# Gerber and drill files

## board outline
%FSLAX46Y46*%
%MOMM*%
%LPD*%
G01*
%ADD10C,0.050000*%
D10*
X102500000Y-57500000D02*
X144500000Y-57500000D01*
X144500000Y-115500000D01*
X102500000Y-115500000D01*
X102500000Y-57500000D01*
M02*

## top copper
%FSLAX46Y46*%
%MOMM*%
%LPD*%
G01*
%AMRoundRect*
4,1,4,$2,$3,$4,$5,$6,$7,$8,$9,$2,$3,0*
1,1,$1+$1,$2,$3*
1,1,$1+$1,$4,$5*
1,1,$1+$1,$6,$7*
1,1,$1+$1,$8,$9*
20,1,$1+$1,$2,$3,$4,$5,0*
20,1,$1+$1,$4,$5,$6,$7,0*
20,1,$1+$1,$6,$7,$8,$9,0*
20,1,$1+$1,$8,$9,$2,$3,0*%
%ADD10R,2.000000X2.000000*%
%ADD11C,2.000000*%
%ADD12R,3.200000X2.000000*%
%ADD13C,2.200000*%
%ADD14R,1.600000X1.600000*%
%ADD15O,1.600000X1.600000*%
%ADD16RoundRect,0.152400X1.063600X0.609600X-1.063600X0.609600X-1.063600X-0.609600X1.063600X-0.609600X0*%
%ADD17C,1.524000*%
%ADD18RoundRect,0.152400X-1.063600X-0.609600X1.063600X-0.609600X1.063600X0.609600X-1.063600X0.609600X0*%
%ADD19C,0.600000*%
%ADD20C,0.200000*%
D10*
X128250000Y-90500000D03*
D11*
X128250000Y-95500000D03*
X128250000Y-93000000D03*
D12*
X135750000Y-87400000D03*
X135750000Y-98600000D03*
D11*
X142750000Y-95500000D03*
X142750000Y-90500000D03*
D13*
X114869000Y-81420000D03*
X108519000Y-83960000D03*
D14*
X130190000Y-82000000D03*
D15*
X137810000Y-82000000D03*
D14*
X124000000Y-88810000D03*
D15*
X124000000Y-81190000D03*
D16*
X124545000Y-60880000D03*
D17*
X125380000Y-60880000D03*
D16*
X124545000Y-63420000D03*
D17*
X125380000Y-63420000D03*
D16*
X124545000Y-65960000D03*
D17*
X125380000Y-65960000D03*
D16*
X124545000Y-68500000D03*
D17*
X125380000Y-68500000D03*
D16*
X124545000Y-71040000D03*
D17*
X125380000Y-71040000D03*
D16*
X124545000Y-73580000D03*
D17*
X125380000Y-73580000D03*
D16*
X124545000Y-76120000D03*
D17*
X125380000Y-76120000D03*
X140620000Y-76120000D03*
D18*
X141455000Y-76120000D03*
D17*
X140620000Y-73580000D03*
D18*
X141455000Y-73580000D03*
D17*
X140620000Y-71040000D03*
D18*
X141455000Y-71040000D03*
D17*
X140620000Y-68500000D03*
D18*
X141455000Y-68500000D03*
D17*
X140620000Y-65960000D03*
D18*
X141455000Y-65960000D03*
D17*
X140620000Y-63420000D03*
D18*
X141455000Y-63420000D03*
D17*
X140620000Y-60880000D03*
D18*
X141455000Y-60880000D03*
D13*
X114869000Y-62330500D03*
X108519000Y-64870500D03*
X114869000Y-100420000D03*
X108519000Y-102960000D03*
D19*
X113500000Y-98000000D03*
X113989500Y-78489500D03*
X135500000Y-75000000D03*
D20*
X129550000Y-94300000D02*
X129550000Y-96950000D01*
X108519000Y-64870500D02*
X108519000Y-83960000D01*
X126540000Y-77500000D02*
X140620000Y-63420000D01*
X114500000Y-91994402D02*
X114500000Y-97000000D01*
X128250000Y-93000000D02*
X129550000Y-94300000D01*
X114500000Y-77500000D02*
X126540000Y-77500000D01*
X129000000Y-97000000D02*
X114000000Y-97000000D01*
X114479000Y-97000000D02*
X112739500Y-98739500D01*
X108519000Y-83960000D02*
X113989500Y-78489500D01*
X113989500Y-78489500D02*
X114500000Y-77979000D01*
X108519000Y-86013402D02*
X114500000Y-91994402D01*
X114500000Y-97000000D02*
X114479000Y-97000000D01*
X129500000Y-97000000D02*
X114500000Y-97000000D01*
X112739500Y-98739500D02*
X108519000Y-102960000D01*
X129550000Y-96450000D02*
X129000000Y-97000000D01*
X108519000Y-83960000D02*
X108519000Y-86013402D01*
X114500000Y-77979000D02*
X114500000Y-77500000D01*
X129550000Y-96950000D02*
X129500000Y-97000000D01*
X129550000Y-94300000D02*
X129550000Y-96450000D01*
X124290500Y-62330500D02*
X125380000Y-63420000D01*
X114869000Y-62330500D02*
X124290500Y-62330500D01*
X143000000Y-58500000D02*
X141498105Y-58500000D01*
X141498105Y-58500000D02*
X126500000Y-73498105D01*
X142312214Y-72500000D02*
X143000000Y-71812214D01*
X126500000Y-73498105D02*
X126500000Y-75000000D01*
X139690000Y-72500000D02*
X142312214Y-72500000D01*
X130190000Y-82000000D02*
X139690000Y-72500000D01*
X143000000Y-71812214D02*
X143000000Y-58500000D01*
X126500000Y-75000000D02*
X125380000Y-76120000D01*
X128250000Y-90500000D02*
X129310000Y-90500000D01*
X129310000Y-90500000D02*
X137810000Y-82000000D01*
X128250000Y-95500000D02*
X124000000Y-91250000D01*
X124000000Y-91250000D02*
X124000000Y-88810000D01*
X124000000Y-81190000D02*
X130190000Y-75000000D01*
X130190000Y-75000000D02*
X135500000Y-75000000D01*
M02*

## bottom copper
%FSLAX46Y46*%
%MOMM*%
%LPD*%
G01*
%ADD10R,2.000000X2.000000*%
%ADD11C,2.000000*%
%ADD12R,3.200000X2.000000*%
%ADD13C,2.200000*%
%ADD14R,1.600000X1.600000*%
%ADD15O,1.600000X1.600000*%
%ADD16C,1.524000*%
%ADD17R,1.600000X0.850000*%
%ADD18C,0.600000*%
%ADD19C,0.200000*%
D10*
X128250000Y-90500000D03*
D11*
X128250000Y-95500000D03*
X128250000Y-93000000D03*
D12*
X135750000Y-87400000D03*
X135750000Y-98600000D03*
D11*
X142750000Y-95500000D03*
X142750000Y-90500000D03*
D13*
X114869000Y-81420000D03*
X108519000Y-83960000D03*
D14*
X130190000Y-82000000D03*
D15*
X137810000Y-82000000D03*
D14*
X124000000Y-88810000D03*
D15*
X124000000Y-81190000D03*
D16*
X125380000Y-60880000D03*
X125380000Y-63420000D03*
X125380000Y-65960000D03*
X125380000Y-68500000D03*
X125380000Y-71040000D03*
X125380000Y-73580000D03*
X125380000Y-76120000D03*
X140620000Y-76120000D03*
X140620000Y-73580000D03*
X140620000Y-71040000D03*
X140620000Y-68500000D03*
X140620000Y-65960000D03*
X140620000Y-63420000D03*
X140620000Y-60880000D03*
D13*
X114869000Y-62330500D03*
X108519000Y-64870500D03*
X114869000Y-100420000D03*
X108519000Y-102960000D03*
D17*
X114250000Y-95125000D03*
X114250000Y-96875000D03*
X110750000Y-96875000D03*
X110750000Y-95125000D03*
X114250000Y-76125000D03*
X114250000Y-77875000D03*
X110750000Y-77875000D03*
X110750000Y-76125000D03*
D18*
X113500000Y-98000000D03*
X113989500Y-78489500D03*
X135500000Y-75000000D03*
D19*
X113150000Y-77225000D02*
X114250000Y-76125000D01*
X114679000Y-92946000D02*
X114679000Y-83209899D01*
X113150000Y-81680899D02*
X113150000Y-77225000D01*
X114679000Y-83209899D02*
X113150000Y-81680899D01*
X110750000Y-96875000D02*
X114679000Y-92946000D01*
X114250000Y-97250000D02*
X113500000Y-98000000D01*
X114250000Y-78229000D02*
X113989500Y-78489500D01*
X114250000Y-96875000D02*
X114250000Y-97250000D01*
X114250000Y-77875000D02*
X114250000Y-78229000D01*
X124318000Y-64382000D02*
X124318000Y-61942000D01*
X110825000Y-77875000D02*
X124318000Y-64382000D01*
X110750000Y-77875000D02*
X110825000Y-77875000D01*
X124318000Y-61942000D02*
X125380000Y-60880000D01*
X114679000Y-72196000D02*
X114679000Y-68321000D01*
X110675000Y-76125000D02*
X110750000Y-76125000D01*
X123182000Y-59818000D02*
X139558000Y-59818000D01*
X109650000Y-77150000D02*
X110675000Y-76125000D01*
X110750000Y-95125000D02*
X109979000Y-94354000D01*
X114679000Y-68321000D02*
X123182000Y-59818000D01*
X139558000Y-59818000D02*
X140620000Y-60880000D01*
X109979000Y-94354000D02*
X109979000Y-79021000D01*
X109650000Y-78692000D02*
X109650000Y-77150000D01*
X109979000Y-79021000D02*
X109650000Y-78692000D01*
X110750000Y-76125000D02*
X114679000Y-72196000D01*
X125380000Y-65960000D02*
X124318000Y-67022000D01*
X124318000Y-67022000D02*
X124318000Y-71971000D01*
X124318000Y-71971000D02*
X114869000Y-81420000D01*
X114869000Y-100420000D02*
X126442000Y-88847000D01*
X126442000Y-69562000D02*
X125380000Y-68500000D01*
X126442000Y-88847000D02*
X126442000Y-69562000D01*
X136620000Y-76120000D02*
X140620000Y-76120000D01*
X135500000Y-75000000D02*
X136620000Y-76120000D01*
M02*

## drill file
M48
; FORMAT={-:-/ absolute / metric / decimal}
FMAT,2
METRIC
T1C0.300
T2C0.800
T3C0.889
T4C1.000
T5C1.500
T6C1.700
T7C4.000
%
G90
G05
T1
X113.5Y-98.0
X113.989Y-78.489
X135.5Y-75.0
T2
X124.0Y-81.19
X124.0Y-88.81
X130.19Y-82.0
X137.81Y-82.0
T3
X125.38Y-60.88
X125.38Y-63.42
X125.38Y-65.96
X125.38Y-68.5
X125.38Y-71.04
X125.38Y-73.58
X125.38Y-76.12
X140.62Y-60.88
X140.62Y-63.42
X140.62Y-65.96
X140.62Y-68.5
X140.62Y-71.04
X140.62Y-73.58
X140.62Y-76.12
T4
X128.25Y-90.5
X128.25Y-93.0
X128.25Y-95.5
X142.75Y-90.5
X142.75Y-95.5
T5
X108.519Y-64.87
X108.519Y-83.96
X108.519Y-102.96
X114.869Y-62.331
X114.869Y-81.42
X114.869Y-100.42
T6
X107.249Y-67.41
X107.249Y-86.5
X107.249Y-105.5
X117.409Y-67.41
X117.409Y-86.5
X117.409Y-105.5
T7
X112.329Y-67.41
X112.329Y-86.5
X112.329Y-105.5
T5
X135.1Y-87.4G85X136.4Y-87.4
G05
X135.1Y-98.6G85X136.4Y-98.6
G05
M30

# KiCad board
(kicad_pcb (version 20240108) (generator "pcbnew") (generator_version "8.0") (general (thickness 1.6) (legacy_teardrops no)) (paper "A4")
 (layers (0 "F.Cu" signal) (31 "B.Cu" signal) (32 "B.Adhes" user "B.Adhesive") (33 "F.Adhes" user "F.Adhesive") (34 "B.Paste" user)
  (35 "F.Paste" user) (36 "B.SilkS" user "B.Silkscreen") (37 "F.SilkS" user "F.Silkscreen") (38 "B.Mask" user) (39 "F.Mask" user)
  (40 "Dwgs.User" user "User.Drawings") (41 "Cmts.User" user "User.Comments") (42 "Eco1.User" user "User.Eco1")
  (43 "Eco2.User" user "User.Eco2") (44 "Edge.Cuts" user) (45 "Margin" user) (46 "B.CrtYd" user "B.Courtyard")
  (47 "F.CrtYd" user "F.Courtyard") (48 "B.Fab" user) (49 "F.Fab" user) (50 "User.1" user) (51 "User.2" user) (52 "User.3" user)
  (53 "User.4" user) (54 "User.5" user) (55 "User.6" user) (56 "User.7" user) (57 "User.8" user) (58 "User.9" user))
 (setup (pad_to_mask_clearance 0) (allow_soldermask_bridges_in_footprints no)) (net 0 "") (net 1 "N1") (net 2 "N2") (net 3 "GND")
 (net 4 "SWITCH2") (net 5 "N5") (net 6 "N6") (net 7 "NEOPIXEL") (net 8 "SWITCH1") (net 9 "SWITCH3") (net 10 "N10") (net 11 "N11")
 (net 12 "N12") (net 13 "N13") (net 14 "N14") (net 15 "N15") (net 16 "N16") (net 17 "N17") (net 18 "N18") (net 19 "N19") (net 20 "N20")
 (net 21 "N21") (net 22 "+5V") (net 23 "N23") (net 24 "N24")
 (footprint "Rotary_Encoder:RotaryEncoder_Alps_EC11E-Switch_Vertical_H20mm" (layer "F.Cu") (at 128.25 90.5)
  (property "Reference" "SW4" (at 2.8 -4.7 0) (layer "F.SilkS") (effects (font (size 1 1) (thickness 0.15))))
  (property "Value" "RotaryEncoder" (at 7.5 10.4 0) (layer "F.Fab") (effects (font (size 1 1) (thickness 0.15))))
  (pad "A" thru_hole rect (at 0 0) (size 2 2) (drill 1) (layers "*.Cu" "*.Mask") (remove_unused_layers no) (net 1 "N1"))
  (pad "B" thru_hole circle (at 0 5) (size 2 2) (drill 1) (layers "*.Cu" "*.Mask") (remove_unused_layers no) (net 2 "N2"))
  (pad "C" thru_hole circle (at 0 2.5) (size 2 2) (drill 1) (layers "*.Cu" "*.Mask") (remove_unused_layers no) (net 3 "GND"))
  (pad "MP" thru_hole rect (at 7.5 -3.1) (size 3.2 2) (drill oval 2.8 1.5) (layers "*.Cu" "*.Mask") (remove_unused_layers no))
  (pad "MP" thru_hole rect (at 7.5 8.1) (size 3.2 2) (drill oval 2.8 1.5) (layers "*.Cu" "*.Mask") (remove_unused_layers no))
  (pad "S1" thru_hole circle (at 14.5 5) (size 2 2) (drill 1) (layers "*.Cu" "*.Mask") (remove_unused_layers no))
  (pad "S2" thru_hole circle (at 14.5 0) (size 2 2) (drill 1) (layers "*.Cu" "*.Mask") (remove_unused_layers no)))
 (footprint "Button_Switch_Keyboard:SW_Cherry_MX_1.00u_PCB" (layer "F.Cu") (at 114.869 81.42)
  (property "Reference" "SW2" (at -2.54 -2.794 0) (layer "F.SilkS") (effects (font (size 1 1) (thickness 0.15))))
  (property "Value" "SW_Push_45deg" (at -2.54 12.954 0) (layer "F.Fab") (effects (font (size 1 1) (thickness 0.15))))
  (pad "" np_thru_hole circle (at -7.62 5.08) (size 1.7 1.7) (drill 1.7) (layers "*.Cu" "*.Mask"))
  (pad "" np_thru_hole circle (at -2.54 5.08) (size 4 4) (drill 4) (layers "*.Cu" "*.Mask"))
  (pad "" np_thru_hole circle (at 2.54 5.08) (size 1.7 1.7) (drill 1.7) (layers "*.Cu" "*.Mask"))
  (pad "1" thru_hole circle (at 0 0) (size 2.2 2.2) (drill 1.5) (layers "*.Cu" "*.Mask") (remove_unused_layers no) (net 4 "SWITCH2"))
  (pad "2" thru_hole circle (at -6.35 2.54) (size 2.2 2.2) (drill 1.5) (layers "*.Cu" "*.Mask") (remove_unused_layers no) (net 3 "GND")))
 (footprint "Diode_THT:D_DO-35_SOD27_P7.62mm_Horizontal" (layer "F.Cu") (at 130.19 82)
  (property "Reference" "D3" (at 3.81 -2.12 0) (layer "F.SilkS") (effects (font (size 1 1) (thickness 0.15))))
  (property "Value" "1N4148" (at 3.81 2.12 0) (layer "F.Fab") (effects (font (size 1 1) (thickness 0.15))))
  (pad "1" thru_hole rect (at 0 0) (size 1.6 1.6) (drill 0.8) (layers "*.Cu" "*.Mask") (remove_unused_layers no) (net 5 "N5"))
  (pad "2" thru_hole oval (at 7.62 0) (size 1.6 1.6) (drill 0.8) (layers "*.Cu" "*.Mask") (remove_unused_layers no) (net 1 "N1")))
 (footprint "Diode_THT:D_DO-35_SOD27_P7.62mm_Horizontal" (layer "F.Cu") (at 124 88.81 90)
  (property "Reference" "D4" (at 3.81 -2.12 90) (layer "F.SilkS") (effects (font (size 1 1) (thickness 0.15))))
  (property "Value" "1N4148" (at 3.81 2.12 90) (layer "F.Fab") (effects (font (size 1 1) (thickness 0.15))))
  (pad "1" thru_hole rect (at 0 0 90) (size 1.6 1.6) (drill 0.8) (layers "*.Cu" "*.Mask") (remove_unused_layers no) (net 2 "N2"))
  (pad "2" thru_hole oval (at 7.62 0 90) (size 1.6 1.6) (drill 0.8) (layers "*.Cu" "*.Mask") (remove_unused_layers no) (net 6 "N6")))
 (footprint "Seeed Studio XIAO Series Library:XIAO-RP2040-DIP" (layer "F.Cu") (at 133 68.5)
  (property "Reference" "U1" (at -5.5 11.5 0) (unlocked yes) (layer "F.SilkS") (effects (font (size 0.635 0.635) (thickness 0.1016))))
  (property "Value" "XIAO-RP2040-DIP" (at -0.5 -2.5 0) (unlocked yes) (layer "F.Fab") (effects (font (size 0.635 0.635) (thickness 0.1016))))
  (pad "1" smd roundrect (at -8.455 -7.62 180) (size 2.432 1.524) (layers "F.Cu" "F.Mask") (roundrect_rratio 0.1) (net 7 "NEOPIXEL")
   (thermal_bridge_angle 45))
  (pad "1" thru_hole circle (at -7.62 -7.62 180) (size 1.524 1.524) (drill 0.889) (layers "*.Cu" "*.Mask") (remove_unused_layers no)
   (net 7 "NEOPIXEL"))
  (pad "2" smd roundrect (at -8.455 -5.08 180) (size 2.432 1.524) (layers "F.Cu" "F.Mask") (roundrect_rratio 0.1) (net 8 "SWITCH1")
   (thermal_bridge_angle 45))
  (pad "2" thru_hole circle (at -7.62 -5.08 180) (size 1.524 1.524) (drill 0.889) (layers "*.Cu" "*.Mask") (remove_unused_layers no)
   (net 8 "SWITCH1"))
  (pad "3" smd roundrect (at -8.455 -2.54 180) (size 2.432 1.524) (layers "F.Cu" "F.Mask") (roundrect_rratio 0.1) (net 4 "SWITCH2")
   (thermal_bridge_angle 45))
  (pad "3" thru_hole circle (at -7.62 -2.54 180) (size 1.524 1.524) (drill 0.889) (layers "*.Cu" "*.Mask") (remove_unused_layers no)
   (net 4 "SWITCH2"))
  (pad "4" smd roundrect (at -8.455 0 180) (size 2.432 1.524) (layers "F.Cu" "F.Mask") (roundrect_rratio 0.1) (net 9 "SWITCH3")
   (thermal_bridge_angle 45))
  (pad "4" thru_hole circle (at -7.62 0 180) (size 1.524 1.524) (drill 0.889) (layers "*.Cu" "*.Mask") (remove_unused_layers no)
   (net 9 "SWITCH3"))
  (pad "5" smd roundrect (at -8.455 2.54 180) (size 2.432 1.524) (layers "F.Cu" "F.Mask") (roundrect_rratio 0.1) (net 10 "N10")
   (thermal_bridge_angle 45))
  (pad "5" thru_hole circle (at -7.62 2.54 180) (size 1.524 1.524) (drill 0.889) (layers "*.Cu" "*.Mask") (remove_unused_layers no)
   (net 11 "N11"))
  (pad "6" smd roundrect (at -8.455 5.08 180) (size 2.432 1.524) (layers "F.Cu" "F.Mask") (roundrect_rratio 0.1) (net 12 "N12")
   (thermal_bridge_angle 45))
  (pad "6" thru_hole circle (at -7.62 5.08 180) (size 1.524 1.524) (drill 0.889) (layers "*.Cu" "*.Mask") (remove_unused_layers no)
   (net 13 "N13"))
  (pad "7" smd roundrect (at -8.455 7.62 180) (size 2.432 1.524) (layers "F.Cu" "F.Mask") (roundrect_rratio 0.1) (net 5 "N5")
   (thermal_bridge_angle 45))
  (pad "7" thru_hole circle (at -7.62 7.62 180) (size 1.524 1.524) (drill 0.889) (layers "*.Cu" "*.Mask") (remove_unused_layers no)
   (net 5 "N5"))
  (pad "8" thru_hole circle (at 7.62 7.62) (size 1.524 1.524) (drill 0.889) (layers "*.Cu" "*.Mask") (remove_unused_layers no) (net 6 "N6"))
  (pad "8" smd roundrect (at 8.455 7.62) (size 2.432 1.524) (layers "F.Cu" "F.Mask") (roundrect_rratio 0.1) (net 6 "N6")
   (thermal_bridge_angle 45))
  (pad "9" thru_hole circle (at 7.62 5.08) (size 1.524 1.524) (drill 0.889) (layers "*.Cu" "*.Mask") (remove_unused_layers no)
   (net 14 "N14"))
  (pad "9" smd roundrect (at 8.455 5.08) (size 2.432 1.524) (layers "F.Cu" "F.Mask") (roundrect_rratio 0.1) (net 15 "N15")
   (thermal_bridge_angle 45))
  (pad "10" thru_hole circle (at 7.62 2.54) (size 1.524 1.524) (drill 0.889) (layers "*.Cu" "*.Mask") (remove_unused_layers no)
   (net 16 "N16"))
  (pad "10" smd roundrect (at 8.455 2.54) (size 2.432 1.524) (layers "F.Cu" "F.Mask") (roundrect_rratio 0.1) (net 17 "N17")
   (thermal_bridge_angle 45))
  (pad "11" thru_hole circle (at 7.62 0) (size 1.524 1.524) (drill 0.889) (layers "*.Cu" "*.Mask") (remove_unused_layers no) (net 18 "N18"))
  (pad "11" smd roundrect (at 8.455 0) (size 2.432 1.524) (layers "F.Cu" "F.Mask") (roundrect_rratio 0.1) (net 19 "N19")
   (thermal_bridge_angle 45))
  (pad "12" thru_hole circle (at 7.62 -2.54) (size 1.524 1.524) (drill 0.889) (layers "*.Cu" "*.Mask") (remove_unused_layers no)
   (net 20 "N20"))
  (pad "12" smd roundrect (at 8.455 -2.54) (size 2.432 1.524) (layers "F.Cu" "F.Mask") (roundrect_rratio 0.1) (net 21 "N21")
   (thermal_bridge_angle 45))
  (pad "13" thru_hole circle (at 7.62 -5.08) (size 1.524 1.524) (drill 0.889) (layers "*.Cu" "*.Mask") (remove_unused_layers no)
   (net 3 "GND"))
  (pad "13" smd roundrect (at 8.455 -5.08) (size 2.432 1.524) (layers "F.Cu" "F.Mask") (roundrect_rratio 0.1) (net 3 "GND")
   (thermal_bridge_angle 45))
  (pad "14" thru_hole circle (at 7.62 -7.62) (size 1.524 1.524) (drill 0.889) (layers "*.Cu" "*.Mask") (remove_unused_layers no)
   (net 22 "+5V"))
  (pad "14" smd roundrect (at 8.455 -7.62) (size 2.432 1.524) (layers "F.Cu" "F.Mask") (roundrect_rratio 0.1) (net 22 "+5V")
   (thermal_bridge_angle 45)))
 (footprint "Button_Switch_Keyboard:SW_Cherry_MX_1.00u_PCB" (layer "F.Cu") (at 114.869 62.3305)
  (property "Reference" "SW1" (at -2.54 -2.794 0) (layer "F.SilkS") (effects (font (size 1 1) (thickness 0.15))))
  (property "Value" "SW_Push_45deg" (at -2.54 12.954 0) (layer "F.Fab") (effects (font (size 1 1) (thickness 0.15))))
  (pad "" np_thru_hole circle (at -7.62 5.08) (size 1.7 1.7) (drill 1.7) (layers "*.Cu" "*.Mask"))
  (pad "" np_thru_hole circle (at -2.54 5.08) (size 4 4) (drill 4) (layers "*.Cu" "*.Mask"))
  (pad "" np_thru_hole circle (at 2.54 5.08) (size 1.7 1.7) (drill 1.7) (layers "*.Cu" "*.Mask"))
  (pad "1" thru_hole circle (at 0 0) (size 2.2 2.2) (drill 1.5) (layers "*.Cu" "*.Mask") (remove_unused_layers no) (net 8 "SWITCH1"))
  (pad "2" thru_hole circle (at -6.35 2.54) (size 2.2 2.2) (drill 1.5) (layers "*.Cu" "*.Mask") (remove_unused_layers no) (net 3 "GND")))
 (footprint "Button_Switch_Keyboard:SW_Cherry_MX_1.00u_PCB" (layer "F.Cu") (at 114.869 100.42)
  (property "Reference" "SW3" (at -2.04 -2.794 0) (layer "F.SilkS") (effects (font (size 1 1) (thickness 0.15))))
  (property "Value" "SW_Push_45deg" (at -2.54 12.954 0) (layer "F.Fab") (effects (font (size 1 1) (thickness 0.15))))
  (pad "" np_thru_hole circle (at -7.62 5.08) (size 1.7 1.7) (drill 1.7) (layers "*.Cu" "*.Mask"))
  (pad "" np_thru_hole circle (at -2.54 5.08) (size 4 4) (drill 4) (layers "*.Cu" "*.Mask"))
  (pad "" np_thru_hole circle (at 2.54 5.08) (size 1.7 1.7) (drill 1.7) (layers "*.Cu" "*.Mask"))
  (pad "1" thru_hole circle (at 0 0) (size 2.2 2.2) (drill 1.5) (layers "*.Cu" "*.Mask") (remove_unused_layers no) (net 9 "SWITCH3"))
  (pad "2" thru_hole circle (at -6.35 2.54) (size 2.2 2.2) (drill 1.5) (layers "*.Cu" "*.Mask") (remove_unused_layers no) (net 3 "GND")))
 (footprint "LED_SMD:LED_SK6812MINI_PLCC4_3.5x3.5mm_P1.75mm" (layer "B.Cu") (at 112.5 96 180)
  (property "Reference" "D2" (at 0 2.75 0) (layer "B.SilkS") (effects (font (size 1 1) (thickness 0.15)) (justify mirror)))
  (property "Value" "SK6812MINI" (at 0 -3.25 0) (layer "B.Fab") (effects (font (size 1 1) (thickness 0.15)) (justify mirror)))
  (pad "1" smd rect (at -1.75 0.875 180) (size 1.6 0.85) (layers "B.Cu" "B.Paste" "B.Mask") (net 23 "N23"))
  (pad "2" smd rect (at -1.75 -0.875 180) (size 1.6 0.85) (layers "B.Cu" "B.Paste" "B.Mask") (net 3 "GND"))
  (pad "3" smd rect (at 1.75 -0.875 180) (size 1.6 0.85) (layers "B.Cu" "B.Paste" "B.Mask") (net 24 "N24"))
  (pad "4" smd rect (at 1.75 0.875 180) (size 1.6 0.85) (layers "B.Cu" "B.Paste" "B.Mask") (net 22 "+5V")))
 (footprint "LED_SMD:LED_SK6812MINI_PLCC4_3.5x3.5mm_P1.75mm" (layer "B.Cu") (at 112.5 77 180)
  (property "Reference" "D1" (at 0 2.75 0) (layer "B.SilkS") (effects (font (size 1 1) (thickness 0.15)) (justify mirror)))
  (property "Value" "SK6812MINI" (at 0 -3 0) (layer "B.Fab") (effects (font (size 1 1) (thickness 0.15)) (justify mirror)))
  (pad "1" smd rect (at -1.75 0.875 180) (size 1.6 0.85) (layers "B.Cu" "B.Paste" "B.Mask") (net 24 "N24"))
  (pad "2" smd rect (at -1.75 -0.875 180) (size 1.6 0.85) (layers "B.Cu" "B.Paste" "B.Mask") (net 3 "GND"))
  (pad "3" smd rect (at 1.75 -0.875 180) (size 1.6 0.85) (layers "B.Cu" "B.Paste" "B.Mask") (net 7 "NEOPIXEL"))
  (pad "4" smd rect (at 1.75 0.875 180) (size 1.6 0.85) (layers "B.Cu" "B.Paste" "B.Mask") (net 22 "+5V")))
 (gr_rect (start 102.5 57.5) (end 144.5 115.5) (stroke (width 0.05) (type default)) (fill none) (layer "Edge.Cuts"))
 (segment (start 113.15 77.225) (end 114.25 76.125) (width 0.2) (layer "B.Cu") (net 24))
 (segment (start 114.679 92.946) (end 114.679 83.209899) (width 0.2) (layer "B.Cu") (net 24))
 (segment (start 113.15 81.680899) (end 113.15 77.225) (width 0.2) (layer "B.Cu") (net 24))
 (segment (start 114.679 83.209899) (end 113.15 81.680899) (width 0.2) (layer "B.Cu") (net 24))
 (segment (start 110.75 96.875) (end 114.679 92.946) (width 0.2) (layer "B.Cu") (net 24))
 (segment (start 129.55 94.3) (end 129.55 96.95) (width 0.2) (layer "F.Cu") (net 3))
 (segment (start 108.519 64.8705) (end 108.519 83.96) (width 0.2) (layer "F.Cu") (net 3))
 (segment (start 126.54 77.5) (end 140.62 63.42) (width 0.2) (layer "F.Cu") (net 3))
 (segment (start 114.5 91.994402) (end 114.5 97) (width 0.2) (layer "F.Cu") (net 3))
 (segment (start 128.25 93) (end 129.55 94.3) (width 0.2) (layer "F.Cu") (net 3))
 (segment (start 114.5 77.5) (end 126.54 77.5) (width 0.2) (layer "F.Cu") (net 3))
 (segment (start 129 97) (end 114 97) (width 0.2) (layer "F.Cu") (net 3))
 (segment (start 114.479 97) (end 112.7395 98.7395) (width 0.2) (layer "F.Cu") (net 3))
 (segment (start 108.519 83.96) (end 113.9895 78.4895) (width 0.2) (layer "F.Cu") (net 3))
 (segment (start 113.9895 78.4895) (end 114.5 77.979) (width 0.2) (layer "F.Cu") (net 3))
 (segment (start 108.519 86.013402) (end 114.5 91.994402) (width 0.2) (layer "F.Cu") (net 3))
 (segment (start 114.5 97) (end 114.479 97) (width 0.2) (layer "F.Cu") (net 3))
 (segment (start 129.5 97) (end 114.5 97) (width 0.2) (layer "F.Cu") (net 3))
 (segment (start 112.7395 98.7395) (end 108.519 102.96) (width 0.2) (layer "F.Cu") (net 3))
 (segment (start 129.55 96.45) (end 129 97) (width 0.2) (layer "F.Cu") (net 3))
 (segment (start 108.519 83.96) (end 108.519 86.013402) (width 0.2) (layer "F.Cu") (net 3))
 (segment (start 114.5 77.979) (end 114.5 77.5) (width 0.2) (layer "F.Cu") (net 3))
 (segment (start 129.55 96.95) (end 129.5 97) (width 0.2) (layer "F.Cu") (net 3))
 (segment (start 129.55 94.3) (end 129.55 96.45) (width 0.2) (layer "F.Cu") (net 3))
 (via (at 113.5 98) (size 0.6) (drill 0.3) (layers "F.Cu" "B.Cu") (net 3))
 (via (at 113.9895 78.4895) (size 0.6) (drill 0.3) (layers "F.Cu" "B.Cu") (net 3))
 (segment (start 114.25 97.25) (end 113.5 98) (width 0.2) (layer "B.Cu") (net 3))
 (segment (start 114.25 78.229) (end 113.9895 78.4895) (width 0.2) (layer "B.Cu") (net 3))
 (segment (start 114.25 96.875) (end 114.25 97.25) (width 0.2) (layer "B.Cu") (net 3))
 (segment (start 114.25 77.875) (end 114.25 78.229) (width 0.2) (layer "B.Cu") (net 3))
 (segment (start 124.318 64.382) (end 124.318 61.942) (width 0.2) (layer "B.Cu") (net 7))
 (segment (start 110.825 77.875) (end 124.318 64.382) (width 0.2) (layer "B.Cu") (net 7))
 (segment (start 110.75 77.875) (end 110.825 77.875) (width 0.2) (layer "B.Cu") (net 7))
 (segment (start 124.318 61.942) (end 125.38 60.88) (width 0.2) (layer "B.Cu") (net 7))
 (segment (start 114.679 72.196) (end 114.679 68.321) (width 0.2) (layer "B.Cu") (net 22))
 (segment (start 110.675 76.125) (end 110.75 76.125) (width 0.2) (layer "B.Cu") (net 22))
 (segment (start 123.182 59.818) (end 139.558 59.818) (width 0.2) (layer "B.Cu") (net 22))
 (segment (start 109.65 77.15) (end 110.675 76.125) (width 0.2) (layer "B.Cu") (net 22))
 (segment (start 110.75 95.125) (end 109.979 94.354) (width 0.2) (layer "B.Cu") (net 22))
 (segment (start 114.679 68.321) (end 123.182 59.818) (width 0.2) (layer "B.Cu") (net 22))
 (segment (start 139.558 59.818) (end 140.62 60.88) (width 0.2) (layer "B.Cu") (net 22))
 (segment (start 109.979 94.354) (end 109.979 79.021) (width 0.2) (layer "B.Cu") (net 22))
 (segment (start 109.65 78.692) (end 109.65 77.15) (width 0.2) (layer "B.Cu") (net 22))
 (segment (start 109.979 79.021) (end 109.65 78.692) (width 0.2) (layer "B.Cu") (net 22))
 (segment (start 110.75 76.125) (end 114.679 72.196) (width 0.2) (layer "B.Cu") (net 22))
 (segment (start 124.2905 62.3305) (end 125.38 63.42) (width 0.2) (layer "F.Cu") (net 8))
 (segment (start 114.869 62.3305) (end 124.2905 62.3305) (width 0.2) (layer "F.Cu") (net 8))
 (segment (start 125.38 65.96) (end 124.318 67.022) (width 0.2) (layer "B.Cu") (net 4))
 (segment (start 124.318 67.022) (end 124.318 71.971) (width 0.2) (layer "B.Cu") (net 4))
 (segment (start 124.318 71.971) (end 114.869 81.42) (width 0.2) (layer "B.Cu") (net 4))
 (segment (start 114.869 100.42) (end 126.442 88.847) (width 0.2) (layer "B.Cu") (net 9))
 (segment (start 126.442 69.562) (end 125.38 68.5) (width 0.2) (layer "B.Cu") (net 9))
 (segment (start 126.442 88.847) (end 126.442 69.562) (width 0.2) (layer "B.Cu") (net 9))
 (segment (start 143 58.5) (end 141.498105 58.5) (width 0.2) (layer "F.Cu") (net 5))
 (segment (start 141.498105 58.5) (end 126.5 73.498105) (width 0.2) (layer "F.Cu") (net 5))
 (segment (start 142.312214 72.5) (end 143 71.812214) (width 0.2) (layer "F.Cu") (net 5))
 (segment (start 126.5 73.498105) (end 126.5 75) (width 0.2) (layer "F.Cu") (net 5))
 (segment (start 139.69 72.5) (end 142.312214 72.5) (width 0.2) (layer "F.Cu") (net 5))
 (segment (start 130.19 82) (end 139.69 72.5) (width 0.2) (layer "F.Cu") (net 5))
 (segment (start 143 71.812214) (end 143 58.5) (width 0.2) (layer "F.Cu") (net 5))
 (segment (start 126.5 75) (end 125.38 76.12) (width 0.2) (layer "F.Cu") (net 5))
 (segment (start 128.25 90.5) (end 129.31 90.5) (width 0.2) (layer "F.Cu") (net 1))
 (segment (start 129.31 90.5) (end 137.81 82) (width 0.2) (layer "F.Cu") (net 1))
 (segment (start 128.25 95.5) (end 124 91.25) (width 0.2) (layer "F.Cu") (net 2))
 (segment (start 124 91.25) (end 124 88.81) (width 0.2) (layer "F.Cu") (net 2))
 (segment (start 124 81.19) (end 130.19 75) (width 0.2) (layer "F.Cu") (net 6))
 (segment (start 130.19 75) (end 135.5 75) (width 0.2) (layer "F.Cu") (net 6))
 (via (at 135.5 75) (size 0.6) (drill 0.3) (layers "F.Cu" "B.Cu") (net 6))
 (segment (start 136.62 76.12) (end 140.62 76.12) (width 0.2) (layer "B.Cu") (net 6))
 (segment (start 135.5 75) (end 136.62 76.12) (width 0.2) (layer "B.Cu") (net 6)))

